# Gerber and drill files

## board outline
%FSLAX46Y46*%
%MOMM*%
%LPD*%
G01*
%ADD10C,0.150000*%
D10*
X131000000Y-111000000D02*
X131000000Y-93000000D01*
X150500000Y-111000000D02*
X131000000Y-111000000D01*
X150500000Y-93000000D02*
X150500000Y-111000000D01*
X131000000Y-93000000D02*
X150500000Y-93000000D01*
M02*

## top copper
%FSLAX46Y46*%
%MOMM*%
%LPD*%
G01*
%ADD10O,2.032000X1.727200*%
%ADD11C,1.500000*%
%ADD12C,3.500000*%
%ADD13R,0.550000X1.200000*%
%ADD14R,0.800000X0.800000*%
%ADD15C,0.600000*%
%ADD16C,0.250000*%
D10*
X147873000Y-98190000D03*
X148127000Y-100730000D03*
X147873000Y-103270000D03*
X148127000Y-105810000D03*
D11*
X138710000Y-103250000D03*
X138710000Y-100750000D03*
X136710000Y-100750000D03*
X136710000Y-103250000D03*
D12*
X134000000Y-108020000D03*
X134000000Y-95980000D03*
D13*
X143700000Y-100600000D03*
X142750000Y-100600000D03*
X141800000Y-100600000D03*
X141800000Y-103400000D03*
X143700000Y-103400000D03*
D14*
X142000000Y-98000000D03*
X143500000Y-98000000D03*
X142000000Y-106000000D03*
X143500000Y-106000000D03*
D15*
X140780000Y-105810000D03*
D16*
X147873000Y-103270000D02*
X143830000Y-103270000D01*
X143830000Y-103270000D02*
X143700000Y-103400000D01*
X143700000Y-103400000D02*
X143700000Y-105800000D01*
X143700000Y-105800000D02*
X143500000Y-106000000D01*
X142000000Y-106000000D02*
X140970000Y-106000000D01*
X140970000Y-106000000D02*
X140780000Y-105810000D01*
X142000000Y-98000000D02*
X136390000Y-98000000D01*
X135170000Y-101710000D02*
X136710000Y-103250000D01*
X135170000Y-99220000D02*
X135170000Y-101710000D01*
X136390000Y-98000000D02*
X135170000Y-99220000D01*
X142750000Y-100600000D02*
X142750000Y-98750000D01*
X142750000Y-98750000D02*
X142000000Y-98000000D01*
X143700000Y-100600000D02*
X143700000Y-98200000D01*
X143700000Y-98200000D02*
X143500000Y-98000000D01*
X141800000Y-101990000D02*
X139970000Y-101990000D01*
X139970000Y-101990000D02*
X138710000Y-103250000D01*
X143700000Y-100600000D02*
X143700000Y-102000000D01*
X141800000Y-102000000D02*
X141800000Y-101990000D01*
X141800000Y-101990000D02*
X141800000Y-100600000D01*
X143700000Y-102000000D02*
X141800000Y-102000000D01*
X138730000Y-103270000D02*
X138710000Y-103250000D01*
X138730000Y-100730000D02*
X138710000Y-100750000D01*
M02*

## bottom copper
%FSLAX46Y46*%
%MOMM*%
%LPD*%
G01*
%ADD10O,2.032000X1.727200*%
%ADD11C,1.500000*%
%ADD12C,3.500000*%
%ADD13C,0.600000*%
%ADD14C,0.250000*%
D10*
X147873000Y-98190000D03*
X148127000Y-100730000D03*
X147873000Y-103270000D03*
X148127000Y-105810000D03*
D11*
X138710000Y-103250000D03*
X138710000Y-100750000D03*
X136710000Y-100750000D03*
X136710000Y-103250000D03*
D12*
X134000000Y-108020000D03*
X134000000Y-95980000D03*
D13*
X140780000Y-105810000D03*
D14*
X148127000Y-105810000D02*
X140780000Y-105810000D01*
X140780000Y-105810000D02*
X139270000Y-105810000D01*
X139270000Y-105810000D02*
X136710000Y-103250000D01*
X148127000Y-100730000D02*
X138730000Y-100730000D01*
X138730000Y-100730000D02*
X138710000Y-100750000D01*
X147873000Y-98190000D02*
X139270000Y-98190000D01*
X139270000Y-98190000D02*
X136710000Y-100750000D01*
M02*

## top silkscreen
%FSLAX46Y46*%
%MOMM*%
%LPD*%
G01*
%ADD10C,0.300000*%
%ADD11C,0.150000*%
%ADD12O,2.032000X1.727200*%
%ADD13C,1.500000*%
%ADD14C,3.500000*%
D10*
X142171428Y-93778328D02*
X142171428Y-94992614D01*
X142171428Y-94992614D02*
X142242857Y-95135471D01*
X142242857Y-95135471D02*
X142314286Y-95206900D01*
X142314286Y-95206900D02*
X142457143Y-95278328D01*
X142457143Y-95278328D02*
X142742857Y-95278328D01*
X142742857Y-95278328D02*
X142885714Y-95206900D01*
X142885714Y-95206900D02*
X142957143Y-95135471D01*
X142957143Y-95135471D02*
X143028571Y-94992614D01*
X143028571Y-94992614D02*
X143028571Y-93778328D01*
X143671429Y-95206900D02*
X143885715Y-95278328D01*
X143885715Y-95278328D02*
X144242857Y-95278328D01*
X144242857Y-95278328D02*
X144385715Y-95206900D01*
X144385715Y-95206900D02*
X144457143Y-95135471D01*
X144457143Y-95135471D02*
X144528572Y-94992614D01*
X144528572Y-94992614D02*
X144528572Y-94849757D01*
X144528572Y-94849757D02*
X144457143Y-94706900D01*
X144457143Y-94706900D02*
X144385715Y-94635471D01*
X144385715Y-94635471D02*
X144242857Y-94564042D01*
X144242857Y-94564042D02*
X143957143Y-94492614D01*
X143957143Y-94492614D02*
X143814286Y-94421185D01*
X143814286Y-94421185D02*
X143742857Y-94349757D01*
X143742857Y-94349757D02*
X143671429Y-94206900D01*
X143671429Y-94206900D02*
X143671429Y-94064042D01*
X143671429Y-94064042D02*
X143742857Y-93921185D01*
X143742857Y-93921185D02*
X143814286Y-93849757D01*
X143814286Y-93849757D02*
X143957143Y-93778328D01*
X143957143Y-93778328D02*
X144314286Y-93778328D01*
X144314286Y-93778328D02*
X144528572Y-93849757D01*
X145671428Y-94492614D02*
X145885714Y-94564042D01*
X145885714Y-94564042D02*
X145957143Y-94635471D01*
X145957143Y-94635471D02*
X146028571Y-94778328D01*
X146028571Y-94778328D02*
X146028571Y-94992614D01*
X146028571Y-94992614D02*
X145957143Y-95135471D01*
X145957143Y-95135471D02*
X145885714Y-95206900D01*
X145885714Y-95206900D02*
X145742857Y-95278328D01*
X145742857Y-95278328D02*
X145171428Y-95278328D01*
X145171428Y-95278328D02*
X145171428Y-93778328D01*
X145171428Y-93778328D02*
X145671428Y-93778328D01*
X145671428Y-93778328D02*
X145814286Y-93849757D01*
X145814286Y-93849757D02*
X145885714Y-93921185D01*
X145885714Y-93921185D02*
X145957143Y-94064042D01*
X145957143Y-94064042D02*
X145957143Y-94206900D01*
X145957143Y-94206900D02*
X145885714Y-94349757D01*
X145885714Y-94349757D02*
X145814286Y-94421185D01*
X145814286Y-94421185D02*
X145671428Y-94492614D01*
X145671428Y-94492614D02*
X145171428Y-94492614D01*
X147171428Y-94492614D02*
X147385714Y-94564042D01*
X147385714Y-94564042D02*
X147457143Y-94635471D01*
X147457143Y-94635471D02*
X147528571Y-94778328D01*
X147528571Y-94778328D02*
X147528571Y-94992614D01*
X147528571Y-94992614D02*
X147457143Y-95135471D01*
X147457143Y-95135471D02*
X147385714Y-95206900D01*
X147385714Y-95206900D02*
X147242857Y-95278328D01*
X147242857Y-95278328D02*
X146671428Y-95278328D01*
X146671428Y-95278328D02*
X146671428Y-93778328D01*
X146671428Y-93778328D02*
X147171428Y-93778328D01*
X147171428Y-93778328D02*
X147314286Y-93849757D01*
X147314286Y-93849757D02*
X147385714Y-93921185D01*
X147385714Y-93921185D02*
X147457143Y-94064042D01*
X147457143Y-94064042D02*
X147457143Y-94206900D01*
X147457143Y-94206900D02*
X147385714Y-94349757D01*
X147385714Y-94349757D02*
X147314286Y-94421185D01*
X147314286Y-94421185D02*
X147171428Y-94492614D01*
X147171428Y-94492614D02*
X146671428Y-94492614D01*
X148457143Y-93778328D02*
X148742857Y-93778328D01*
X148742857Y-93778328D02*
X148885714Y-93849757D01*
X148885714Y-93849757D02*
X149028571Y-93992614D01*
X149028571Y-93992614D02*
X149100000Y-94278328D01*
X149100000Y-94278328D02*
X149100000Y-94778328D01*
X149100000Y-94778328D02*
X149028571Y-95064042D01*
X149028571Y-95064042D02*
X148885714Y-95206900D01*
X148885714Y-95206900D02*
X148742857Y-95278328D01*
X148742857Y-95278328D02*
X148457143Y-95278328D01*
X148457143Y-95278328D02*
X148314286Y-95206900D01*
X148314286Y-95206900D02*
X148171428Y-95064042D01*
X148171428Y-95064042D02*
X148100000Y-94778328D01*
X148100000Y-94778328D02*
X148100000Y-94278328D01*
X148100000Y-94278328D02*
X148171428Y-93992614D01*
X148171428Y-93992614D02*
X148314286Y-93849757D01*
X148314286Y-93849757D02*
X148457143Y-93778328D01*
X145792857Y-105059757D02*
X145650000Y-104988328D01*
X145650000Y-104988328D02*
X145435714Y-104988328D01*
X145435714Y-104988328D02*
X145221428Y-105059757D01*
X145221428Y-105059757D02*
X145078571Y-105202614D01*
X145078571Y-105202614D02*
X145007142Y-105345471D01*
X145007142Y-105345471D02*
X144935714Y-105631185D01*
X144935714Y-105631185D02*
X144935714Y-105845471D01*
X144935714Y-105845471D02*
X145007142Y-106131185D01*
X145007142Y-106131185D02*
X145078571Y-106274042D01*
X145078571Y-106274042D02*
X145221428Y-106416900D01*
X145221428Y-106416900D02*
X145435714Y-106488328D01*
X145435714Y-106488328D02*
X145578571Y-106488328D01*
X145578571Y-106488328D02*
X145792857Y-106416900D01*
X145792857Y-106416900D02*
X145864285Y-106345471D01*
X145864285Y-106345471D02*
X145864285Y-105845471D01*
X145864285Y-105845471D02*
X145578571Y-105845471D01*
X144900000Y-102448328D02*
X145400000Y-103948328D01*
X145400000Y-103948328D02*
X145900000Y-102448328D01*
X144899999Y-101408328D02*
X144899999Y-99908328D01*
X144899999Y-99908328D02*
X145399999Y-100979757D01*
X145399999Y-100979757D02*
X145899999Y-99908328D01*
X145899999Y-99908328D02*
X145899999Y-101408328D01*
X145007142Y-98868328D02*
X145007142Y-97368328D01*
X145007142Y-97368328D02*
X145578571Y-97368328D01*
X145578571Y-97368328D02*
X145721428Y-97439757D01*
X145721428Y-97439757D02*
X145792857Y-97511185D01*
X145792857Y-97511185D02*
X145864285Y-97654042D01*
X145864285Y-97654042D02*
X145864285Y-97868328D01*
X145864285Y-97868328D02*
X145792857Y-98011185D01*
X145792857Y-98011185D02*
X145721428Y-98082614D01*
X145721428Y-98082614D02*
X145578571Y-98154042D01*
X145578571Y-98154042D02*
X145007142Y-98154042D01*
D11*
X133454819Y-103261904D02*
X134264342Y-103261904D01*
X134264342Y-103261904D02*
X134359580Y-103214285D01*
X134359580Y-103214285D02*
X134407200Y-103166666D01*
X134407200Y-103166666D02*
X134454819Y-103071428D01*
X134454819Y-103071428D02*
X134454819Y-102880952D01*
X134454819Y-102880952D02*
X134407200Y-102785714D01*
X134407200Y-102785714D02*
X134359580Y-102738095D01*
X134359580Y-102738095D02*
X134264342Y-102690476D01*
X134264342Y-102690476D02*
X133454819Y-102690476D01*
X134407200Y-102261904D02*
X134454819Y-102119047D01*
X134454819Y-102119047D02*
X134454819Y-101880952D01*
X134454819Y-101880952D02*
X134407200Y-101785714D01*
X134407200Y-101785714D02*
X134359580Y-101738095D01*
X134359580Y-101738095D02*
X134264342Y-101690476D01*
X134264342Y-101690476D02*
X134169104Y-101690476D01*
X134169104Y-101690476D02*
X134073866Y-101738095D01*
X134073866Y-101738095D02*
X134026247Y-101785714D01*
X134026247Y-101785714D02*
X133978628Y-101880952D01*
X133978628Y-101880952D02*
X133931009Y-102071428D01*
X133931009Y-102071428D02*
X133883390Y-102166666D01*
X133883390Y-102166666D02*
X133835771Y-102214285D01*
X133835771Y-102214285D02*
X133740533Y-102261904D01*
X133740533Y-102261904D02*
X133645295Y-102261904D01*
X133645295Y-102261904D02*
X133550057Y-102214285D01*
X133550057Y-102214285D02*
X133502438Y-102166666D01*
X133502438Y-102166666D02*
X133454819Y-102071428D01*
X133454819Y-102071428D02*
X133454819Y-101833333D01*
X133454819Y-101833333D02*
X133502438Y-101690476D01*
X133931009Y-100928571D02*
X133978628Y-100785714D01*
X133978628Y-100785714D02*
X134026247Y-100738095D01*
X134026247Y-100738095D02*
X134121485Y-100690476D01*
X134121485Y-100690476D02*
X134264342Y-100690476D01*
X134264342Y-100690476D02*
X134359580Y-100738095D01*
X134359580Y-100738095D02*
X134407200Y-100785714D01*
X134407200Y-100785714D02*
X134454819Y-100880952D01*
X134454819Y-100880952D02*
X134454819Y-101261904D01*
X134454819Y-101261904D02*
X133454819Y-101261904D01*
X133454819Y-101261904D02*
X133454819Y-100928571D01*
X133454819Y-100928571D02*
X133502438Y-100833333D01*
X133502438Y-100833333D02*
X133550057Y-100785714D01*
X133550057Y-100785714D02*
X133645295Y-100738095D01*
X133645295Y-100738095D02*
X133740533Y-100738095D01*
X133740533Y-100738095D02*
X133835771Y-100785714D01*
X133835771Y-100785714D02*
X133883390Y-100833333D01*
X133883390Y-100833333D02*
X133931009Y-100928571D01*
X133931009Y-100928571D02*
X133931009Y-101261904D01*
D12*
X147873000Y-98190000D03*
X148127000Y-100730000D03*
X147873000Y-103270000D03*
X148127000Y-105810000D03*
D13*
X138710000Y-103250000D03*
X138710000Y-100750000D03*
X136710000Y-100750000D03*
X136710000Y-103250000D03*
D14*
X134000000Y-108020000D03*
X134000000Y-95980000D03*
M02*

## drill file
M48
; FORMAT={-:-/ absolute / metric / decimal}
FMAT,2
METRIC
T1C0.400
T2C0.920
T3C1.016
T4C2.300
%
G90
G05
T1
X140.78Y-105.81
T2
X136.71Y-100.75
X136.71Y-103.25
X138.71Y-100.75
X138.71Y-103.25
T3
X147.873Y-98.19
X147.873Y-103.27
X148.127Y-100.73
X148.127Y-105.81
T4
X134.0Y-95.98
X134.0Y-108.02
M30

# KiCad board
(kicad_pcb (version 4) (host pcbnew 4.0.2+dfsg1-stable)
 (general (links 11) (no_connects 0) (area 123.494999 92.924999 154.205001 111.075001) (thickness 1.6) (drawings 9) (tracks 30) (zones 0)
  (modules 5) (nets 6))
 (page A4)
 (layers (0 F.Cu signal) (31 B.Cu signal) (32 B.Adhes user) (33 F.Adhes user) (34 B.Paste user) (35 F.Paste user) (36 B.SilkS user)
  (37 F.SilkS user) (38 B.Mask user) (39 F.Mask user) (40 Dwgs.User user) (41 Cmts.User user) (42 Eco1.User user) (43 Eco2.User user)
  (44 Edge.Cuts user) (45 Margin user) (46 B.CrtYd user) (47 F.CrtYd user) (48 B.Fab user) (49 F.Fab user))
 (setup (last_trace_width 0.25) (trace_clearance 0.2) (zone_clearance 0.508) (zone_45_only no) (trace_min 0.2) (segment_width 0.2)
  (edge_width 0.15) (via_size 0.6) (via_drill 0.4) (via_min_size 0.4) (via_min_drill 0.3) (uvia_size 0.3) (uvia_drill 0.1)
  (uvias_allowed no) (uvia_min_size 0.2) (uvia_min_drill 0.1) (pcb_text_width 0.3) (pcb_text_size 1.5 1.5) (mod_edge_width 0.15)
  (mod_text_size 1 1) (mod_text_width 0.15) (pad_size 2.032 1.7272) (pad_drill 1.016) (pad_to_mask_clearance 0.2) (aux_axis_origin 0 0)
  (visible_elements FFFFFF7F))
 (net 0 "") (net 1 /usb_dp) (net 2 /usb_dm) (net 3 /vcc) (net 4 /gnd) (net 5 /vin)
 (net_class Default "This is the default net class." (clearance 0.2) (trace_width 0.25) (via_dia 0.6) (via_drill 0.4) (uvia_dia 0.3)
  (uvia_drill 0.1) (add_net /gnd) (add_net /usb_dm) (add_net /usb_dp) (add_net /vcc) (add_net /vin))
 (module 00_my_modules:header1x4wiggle (layer F.Cu) (at 148 102)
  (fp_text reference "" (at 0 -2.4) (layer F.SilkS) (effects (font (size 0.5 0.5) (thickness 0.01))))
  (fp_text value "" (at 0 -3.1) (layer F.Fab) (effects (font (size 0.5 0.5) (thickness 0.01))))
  (pad 1 thru_hole oval (at -0.127 -3.81) (size 2.032 1.7272) (drill 1.016) (layers *.Cu *.Mask F.SilkS) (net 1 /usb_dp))
  (pad 2 thru_hole oval (at 0.127 -1.27) (size 2.032 1.7272) (drill 1.016) (layers *.Cu *.Mask F.SilkS) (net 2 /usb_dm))
  (pad 3 thru_hole oval (at -0.127 1.27) (size 2.032 1.7272) (drill 1.016) (layers *.Cu *.Mask F.SilkS) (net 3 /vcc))
  (pad 4 thru_hole oval (at 0.127 3.81) (size 2.032 1.7272) (drill 1.016) (layers *.Cu *.Mask F.SilkS) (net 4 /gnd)))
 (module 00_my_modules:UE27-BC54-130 (layer F.Cu) (at 134 102 270)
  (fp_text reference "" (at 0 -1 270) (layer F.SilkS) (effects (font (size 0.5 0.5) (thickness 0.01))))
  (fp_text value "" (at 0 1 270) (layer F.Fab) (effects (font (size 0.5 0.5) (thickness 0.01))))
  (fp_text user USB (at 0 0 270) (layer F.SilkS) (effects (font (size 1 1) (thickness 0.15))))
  (pad V thru_hole circle (at 1.25 -4.71 270) (size 1.5 1.5) (drill 0.92) (layers *.Cu *.Mask F.SilkS) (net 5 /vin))
  (pad - thru_hole circle (at -1.25 -4.71 270) (size 1.5 1.5) (drill 0.92) (layers *.Cu *.Mask F.SilkS) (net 2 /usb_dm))
  (pad + thru_hole circle (at -1.25 -2.71 270) (size 1.5 1.5) (drill 0.92) (layers *.Cu *.Mask F.SilkS) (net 1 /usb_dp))
  (pad G thru_hole circle (at 1.25 -2.71 270) (size 1.5 1.5) (drill 0.92) (layers *.Cu *.Mask F.SilkS) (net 4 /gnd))
  (pad X thru_hole circle (at 6.02 0 270) (size 3.5 3.5) (drill 2.3) (layers *.Cu *.Mask F.SilkS))
  (pad X thru_hole circle (at -6.02 0 270) (size 3.5 3.5) (drill 2.3) (layers *.Cu *.Mask F.SilkS)))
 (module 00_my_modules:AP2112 (layer F.Cu) (at 142.75 102 270)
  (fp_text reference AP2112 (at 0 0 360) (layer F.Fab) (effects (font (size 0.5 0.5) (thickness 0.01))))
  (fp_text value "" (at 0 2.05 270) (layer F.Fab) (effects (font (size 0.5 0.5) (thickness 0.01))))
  (pad VIN smd rect (at -1.4 -0.95 270) (size 1.2 0.55) (layers F.Cu F.Paste F.Mask) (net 5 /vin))
  (pad GND smd rect (at -1.4 0 270) (size 1.2 0.55) (layers F.Cu F.Paste F.Mask) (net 4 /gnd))
  (pad EN smd rect (at -1.4 0.95 270) (size 1.2 0.55) (layers F.Cu F.Paste F.Mask) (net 5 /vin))
  (pad NC smd rect (at 1.4 0.95 270) (size 1.2 0.55) (layers F.Cu F.Paste F.Mask))
  (pad VOUT smd rect (at 1.4 -0.95 270) (size 1.2 0.55) (layers F.Cu F.Paste F.Mask) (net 3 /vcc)))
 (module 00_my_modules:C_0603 (layer F.Cu) (at 142.75 98)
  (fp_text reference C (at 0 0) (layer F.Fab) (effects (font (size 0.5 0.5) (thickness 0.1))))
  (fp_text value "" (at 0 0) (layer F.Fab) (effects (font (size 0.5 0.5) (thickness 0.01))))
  (pad 1 smd rect (at -0.75 0) (size 0.8 0.8) (layers F.Cu F.Paste F.Mask) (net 4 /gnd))
  (pad 2 smd rect (at 0.75 0) (size 0.8 0.8) (layers F.Cu F.Paste F.Mask) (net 5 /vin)))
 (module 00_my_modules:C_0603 (layer F.Cu) (at 142.75 106)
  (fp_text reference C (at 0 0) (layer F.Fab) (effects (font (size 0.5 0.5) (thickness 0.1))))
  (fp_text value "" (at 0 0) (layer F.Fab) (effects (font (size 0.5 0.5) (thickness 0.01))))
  (pad 1 smd rect (at -0.75 0) (size 0.8 0.8) (layers F.Cu F.Paste F.Mask) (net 4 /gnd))
  (pad 2 smd rect (at 0.75 0) (size 0.8 0.8) (layers F.Cu F.Paste F.Mask) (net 3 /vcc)))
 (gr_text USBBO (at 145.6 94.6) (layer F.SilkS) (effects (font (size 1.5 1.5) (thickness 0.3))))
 (gr_line (start 131 111) (end 131 93) (angle 90) (layer Edge.Cuts) (width 0.15))
 (gr_line (start 150.5 111) (end 131 111) (angle 90) (layer Edge.Cuts) (width 0.15))
 (gr_line (start 150.5 93) (end 150.5 111) (angle 90) (layer Edge.Cuts) (width 0.15))
 (gr_line (start 131 93) (end 150.5 93) (angle 90) (layer Edge.Cuts) (width 0.15))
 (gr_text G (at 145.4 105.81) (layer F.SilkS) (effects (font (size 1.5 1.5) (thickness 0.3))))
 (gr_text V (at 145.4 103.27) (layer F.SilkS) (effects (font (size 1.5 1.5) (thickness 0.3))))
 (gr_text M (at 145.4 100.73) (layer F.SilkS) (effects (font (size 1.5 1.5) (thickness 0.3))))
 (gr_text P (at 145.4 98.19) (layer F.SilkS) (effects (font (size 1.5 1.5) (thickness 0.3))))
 (segment (start 147.873 103.27) (end 143.83 103.27) (width 0.25) (layer F.Cu) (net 3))
 (segment (start 143.83 103.27) (end 143.7 103.4) (width 0.25) (layer F.Cu) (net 3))
 (segment (start 143.7 103.4) (end 143.7 105.8) (width 0.25) (layer F.Cu) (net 3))
 (segment (start 143.7 105.8) (end 143.5 106) (width 0.25) (layer F.Cu) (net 3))
 (via (at 140.78 105.81) (size 0.6) (drill 0.4) (layers F.Cu B.Cu) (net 4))
 (segment (start 142 106) (end 140.97 106) (width 0.25) (layer F.Cu) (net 4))
 (segment (start 140.97 106) (end 140.78 105.81) (width 0.25) (layer F.Cu) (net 4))
 (segment (start 142 98) (end 136.39 98) (width 0.25) (layer F.Cu) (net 4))
 (segment (start 135.17 101.71) (end 136.71 103.25) (width 0.25) (layer F.Cu) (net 4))
 (segment (start 135.17 99.22) (end 135.17 101.71) (width 0.25) (layer F.Cu) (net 4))
 (segment (start 136.39 98) (end 135.17 99.22) (width 0.25) (layer F.Cu) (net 4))
 (segment (start 148.127 105.81) (end 140.78 105.81) (width 0.25) (layer B.Cu) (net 4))
 (segment (start 140.78 105.81) (end 139.27 105.81) (width 0.25) (layer B.Cu) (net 4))
 (segment (start 139.27 105.81) (end 136.71 103.25) (width 0.25) (layer B.Cu) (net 4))
 (segment (start 142.75 100.6) (end 142.75 98.75) (width 0.25) (layer F.Cu) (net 4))
 (segment (start 142.75 98.75) (end 142 98) (width 0.25) (layer F.Cu) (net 4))
 (segment (start 143.7 100.6) (end 143.7 98.2) (width 0.25) (layer F.Cu) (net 5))
 (segment (start 143.7 98.2) (end 143.5 98) (width 0.25) (layer F.Cu) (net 5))
 (segment (start 141.8 101.99) (end 139.97 101.99) (width 0.25) (layer F.Cu) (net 5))
 (segment (start 139.97 101.99) (end 138.71 103.25) (width 0.25) (layer F.Cu) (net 5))
 (segment (start 143.7 100.6) (end 143.7 102) (width 0.25) (layer F.Cu) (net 5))
 (segment (start 141.8 102) (end 141.8 101.99) (width 0.25) (layer F.Cu) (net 5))
 (segment (start 141.8 101.99) (end 141.8 100.6) (width 0.25) (layer F.Cu) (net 5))
 (segment (start 143.7 102) (end 141.8 102) (width 0.25) (layer F.Cu) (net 5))
 (segment (start 138.73 103.27) (end 138.71 103.25) (width 0.25) (layer F.Cu) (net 5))
 (segment (start 148.127 100.73) (end 138.73 100.73) (width 0.25) (layer B.Cu) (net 2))
 (segment (start 138.73 100.73) (end 138.71 100.75) (width 0.25) (layer B.Cu) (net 2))
 (segment (start 138.73 100.73) (end 138.71 100.75) (width 0.25) (layer F.Cu) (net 2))
 (segment (start 147.873 98.19) (end 139.27 98.19) (width 0.25) (layer B.Cu) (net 1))
 (segment (start 139.27 98.19) (end 136.71 100.75) (width 0.25) (layer B.Cu) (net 1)))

